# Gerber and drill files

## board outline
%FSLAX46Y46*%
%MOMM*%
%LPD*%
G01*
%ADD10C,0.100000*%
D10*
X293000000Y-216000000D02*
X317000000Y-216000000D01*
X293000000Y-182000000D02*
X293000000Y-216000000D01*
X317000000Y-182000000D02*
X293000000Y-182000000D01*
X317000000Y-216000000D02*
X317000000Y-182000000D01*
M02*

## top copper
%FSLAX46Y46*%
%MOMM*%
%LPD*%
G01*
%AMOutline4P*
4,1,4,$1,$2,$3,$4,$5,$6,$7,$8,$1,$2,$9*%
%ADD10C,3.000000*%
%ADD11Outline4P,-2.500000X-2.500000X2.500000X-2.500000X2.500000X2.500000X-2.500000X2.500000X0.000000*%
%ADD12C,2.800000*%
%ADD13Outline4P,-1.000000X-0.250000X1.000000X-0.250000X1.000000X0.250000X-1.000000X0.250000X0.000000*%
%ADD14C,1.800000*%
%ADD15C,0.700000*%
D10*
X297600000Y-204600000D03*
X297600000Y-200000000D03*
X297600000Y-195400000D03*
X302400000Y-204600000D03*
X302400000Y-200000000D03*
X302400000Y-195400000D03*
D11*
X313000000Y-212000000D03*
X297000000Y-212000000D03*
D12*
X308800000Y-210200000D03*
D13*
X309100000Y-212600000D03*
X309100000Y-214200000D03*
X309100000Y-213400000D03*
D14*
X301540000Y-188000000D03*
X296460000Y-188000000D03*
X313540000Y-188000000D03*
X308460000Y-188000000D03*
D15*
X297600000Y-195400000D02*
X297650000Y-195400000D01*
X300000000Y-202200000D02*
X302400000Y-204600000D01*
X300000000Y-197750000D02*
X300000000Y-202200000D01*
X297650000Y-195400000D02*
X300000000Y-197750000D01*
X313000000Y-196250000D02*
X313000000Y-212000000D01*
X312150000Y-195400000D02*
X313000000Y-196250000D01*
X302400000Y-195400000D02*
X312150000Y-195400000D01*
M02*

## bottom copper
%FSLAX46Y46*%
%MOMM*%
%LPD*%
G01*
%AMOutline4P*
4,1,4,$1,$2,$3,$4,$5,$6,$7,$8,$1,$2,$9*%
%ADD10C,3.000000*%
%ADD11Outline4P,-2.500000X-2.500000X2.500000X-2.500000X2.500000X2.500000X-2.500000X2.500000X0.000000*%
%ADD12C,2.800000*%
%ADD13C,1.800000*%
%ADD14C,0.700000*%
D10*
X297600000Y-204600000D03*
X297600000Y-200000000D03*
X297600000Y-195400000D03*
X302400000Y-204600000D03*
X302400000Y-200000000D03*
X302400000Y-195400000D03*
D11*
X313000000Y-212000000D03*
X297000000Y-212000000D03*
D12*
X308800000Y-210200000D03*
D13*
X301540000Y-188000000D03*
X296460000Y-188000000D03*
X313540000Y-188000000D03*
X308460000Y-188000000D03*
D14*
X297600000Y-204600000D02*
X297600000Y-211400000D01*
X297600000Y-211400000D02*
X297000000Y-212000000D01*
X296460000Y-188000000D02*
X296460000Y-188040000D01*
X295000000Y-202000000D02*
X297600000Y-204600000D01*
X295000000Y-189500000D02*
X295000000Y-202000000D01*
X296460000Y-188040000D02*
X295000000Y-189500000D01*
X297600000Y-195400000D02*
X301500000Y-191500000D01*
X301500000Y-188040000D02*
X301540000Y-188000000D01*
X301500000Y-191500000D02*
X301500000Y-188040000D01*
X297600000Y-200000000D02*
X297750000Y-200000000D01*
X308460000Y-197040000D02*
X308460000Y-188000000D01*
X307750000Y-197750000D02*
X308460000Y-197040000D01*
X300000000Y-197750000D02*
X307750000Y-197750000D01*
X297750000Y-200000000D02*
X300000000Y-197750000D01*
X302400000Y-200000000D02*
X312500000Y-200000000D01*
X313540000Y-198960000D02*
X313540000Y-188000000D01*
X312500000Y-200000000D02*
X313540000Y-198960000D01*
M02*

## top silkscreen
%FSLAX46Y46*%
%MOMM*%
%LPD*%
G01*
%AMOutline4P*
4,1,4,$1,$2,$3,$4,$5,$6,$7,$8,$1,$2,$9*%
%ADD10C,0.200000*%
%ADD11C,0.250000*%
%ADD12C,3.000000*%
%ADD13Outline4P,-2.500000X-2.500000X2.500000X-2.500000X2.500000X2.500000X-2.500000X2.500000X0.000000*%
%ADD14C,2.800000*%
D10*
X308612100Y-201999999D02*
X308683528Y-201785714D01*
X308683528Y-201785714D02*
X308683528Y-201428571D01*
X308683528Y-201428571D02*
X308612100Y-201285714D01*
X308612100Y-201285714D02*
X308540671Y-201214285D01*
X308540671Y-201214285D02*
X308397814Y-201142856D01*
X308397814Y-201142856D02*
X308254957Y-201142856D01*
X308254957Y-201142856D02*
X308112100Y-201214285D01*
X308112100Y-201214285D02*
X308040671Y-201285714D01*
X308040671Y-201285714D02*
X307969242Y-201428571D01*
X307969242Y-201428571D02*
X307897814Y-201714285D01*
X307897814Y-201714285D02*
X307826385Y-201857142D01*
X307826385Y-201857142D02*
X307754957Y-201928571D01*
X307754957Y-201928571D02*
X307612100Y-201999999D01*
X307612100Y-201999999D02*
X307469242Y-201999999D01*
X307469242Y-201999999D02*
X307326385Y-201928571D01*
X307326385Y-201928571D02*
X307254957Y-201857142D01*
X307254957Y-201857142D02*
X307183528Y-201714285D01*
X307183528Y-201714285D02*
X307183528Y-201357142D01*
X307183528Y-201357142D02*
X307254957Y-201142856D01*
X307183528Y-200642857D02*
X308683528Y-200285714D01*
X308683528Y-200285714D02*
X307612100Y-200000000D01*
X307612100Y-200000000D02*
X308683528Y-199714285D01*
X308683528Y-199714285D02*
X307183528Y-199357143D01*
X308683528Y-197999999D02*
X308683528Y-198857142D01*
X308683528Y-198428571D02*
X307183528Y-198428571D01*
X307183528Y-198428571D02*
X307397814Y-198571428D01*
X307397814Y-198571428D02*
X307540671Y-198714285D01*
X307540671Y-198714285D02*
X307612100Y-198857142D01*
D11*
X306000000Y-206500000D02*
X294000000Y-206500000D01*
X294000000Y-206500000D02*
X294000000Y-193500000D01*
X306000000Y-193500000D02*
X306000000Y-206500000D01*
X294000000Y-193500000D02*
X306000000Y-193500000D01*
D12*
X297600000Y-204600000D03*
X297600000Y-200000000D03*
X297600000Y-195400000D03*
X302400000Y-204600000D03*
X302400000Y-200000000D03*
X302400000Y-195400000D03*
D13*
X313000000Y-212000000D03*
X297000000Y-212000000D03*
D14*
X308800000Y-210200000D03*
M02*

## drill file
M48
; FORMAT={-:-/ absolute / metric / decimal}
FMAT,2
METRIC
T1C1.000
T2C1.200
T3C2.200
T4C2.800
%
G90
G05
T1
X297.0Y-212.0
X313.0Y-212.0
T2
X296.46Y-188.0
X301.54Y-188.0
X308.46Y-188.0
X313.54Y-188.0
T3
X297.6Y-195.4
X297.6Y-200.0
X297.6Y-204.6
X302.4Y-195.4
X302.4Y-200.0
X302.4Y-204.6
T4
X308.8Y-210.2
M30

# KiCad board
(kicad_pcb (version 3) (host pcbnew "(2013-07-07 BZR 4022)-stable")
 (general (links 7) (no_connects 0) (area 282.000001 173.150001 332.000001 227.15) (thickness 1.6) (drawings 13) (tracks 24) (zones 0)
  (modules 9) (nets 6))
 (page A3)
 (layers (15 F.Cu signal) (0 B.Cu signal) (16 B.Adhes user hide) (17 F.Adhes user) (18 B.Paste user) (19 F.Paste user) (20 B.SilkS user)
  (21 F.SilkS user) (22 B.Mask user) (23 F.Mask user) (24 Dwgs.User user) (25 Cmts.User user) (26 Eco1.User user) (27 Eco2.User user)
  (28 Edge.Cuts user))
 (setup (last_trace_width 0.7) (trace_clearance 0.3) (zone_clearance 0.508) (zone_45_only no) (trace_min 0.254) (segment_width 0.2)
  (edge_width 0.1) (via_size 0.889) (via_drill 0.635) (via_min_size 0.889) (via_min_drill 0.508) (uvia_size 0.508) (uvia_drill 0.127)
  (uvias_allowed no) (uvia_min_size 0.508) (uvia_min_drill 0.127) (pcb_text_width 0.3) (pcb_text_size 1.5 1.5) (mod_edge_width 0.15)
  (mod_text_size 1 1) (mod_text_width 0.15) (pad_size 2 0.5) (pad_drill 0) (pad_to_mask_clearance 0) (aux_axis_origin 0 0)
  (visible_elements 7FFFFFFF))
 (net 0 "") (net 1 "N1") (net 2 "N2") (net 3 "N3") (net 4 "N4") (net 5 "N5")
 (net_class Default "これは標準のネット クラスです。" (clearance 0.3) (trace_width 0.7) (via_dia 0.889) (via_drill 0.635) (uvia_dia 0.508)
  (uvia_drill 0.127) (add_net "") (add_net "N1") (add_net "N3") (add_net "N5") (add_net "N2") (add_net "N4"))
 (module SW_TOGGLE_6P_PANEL (layer F.Cu) (at 300 200)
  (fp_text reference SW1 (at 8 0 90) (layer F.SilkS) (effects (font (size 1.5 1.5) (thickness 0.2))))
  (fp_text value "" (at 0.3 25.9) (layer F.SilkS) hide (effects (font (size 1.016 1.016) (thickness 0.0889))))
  (fp_line (start 6 6.5) (end -6 6.5) (layer F.SilkS) (width 0.25))
  (fp_line (start -6 6.5) (end -6 -6.5) (layer F.SilkS) (width 0.25))
  (fp_line (start 6 -6.5) (end 6 6.5) (layer F.SilkS) (width 0.25))
  (fp_line (start -6 -6.5) (end 6 -6.5) (layer F.SilkS) (width 0.25))
  (pad 1 thru_hole circle (at -2.4 4.6) (size 3 3) (drill 2.2) (layers *.Cu *.Mask F.SilkS) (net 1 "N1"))
  (pad 2 thru_hole circle (at -2.4 0) (size 3 3) (drill 2.2) (layers *.Cu *.Mask F.SilkS) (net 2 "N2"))
  (pad 3 thru_hole circle (at -2.4 -4.6) (size 3 3) (drill 2.2) (layers *.Cu *.Mask F.SilkS) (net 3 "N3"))
  (pad 4 thru_hole circle (at 2.4 4.6) (size 3 3) (drill 2.2) (layers *.Cu *.Mask F.SilkS) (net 3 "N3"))
  (pad 5 thru_hole circle (at 2.4 0) (size 3 3) (drill 2.2) (layers *.Cu *.Mask F.SilkS) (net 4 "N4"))
  (pad 6 thru_hole circle (at 2.4 -4.6) (size 3 3) (drill 2.2) (layers *.Cu *.Mask F.SilkS) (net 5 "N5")))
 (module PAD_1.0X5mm (layer F.Cu) (at 313 212)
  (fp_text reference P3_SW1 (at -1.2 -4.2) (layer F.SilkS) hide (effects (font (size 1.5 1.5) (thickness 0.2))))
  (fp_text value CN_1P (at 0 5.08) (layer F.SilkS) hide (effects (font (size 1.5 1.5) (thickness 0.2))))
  (pad 1 thru_hole trapezoid (at 0 0) (size 5 5) (drill 1) (layers *.Cu *.Mask F.SilkS) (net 5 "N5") (clearance 0.3)))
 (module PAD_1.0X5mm (layer F.Cu) (at 297 212)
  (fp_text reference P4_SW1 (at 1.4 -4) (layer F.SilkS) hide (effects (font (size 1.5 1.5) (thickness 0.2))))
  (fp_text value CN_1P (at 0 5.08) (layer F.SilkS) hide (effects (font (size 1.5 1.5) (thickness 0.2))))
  (pad 1 thru_hole trapezoid (at 0 0) (size 5 5) (drill 1) (layers *.Cu *.Mask F.SilkS) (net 1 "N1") (clearance 0.3)))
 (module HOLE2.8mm (layer F.Cu) (at 308.8 210.2)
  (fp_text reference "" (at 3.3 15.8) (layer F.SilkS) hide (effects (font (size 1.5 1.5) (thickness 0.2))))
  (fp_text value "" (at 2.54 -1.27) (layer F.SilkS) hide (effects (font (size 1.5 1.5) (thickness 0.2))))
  (pad "" thru_hole circle (at 0 0) (size 2.8 2.8) (drill 2.8) (layers *.Cu *.Mask F.SilkS) (clearance 0.3)))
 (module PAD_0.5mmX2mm (layer F.Cu) (at 309.1 212.6)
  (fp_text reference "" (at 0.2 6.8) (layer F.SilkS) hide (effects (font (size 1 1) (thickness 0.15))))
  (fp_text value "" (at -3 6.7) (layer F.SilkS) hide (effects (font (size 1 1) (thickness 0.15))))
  (pad 1 smd trapezoid (at 0 0) (size 2 0.5) (layers F.Cu F.Paste F.Mask)))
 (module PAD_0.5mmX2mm (layer F.Cu) (at 309.1 214.2)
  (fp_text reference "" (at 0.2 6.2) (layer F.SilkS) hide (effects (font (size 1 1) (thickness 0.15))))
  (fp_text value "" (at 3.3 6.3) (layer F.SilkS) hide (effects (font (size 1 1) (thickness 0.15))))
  (pad 1 smd trapezoid (at 0 0) (size 2 0.5) (layers F.Cu F.Paste F.Mask)))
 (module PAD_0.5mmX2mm (layer F.Cu) (at 309.1 213.4)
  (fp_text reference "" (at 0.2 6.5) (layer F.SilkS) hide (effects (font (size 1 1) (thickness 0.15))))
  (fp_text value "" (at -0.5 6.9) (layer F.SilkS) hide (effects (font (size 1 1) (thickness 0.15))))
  (pad 1 smd trapezoid (at 0 0) (size 2 0.5) (layers F.Cu F.Paste F.Mask)))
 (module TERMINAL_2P (layer B.Cu) (at 299 188 180)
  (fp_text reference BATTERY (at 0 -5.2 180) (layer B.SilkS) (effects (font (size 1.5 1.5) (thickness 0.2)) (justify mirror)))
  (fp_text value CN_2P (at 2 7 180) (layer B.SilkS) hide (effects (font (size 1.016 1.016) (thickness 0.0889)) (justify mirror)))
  (pad 1 thru_hole circle (at -2.54 0 180) (size 1.8 1.8) (drill 1.2) (layers *.Cu *.Mask B.SilkS) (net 3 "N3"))
  (pad 2 thru_hole circle (at 2.54 0 180) (size 1.8 1.8) (drill 1.2) (layers *.Cu *.Mask B.SilkS) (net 1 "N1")))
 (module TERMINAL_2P (layer B.Cu) (at 311 188 180)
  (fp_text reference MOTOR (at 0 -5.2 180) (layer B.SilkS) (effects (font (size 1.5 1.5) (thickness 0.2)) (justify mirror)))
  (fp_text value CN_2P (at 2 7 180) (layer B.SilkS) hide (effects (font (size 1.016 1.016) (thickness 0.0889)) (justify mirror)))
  (pad 1 thru_hole circle (at -2.54 0 180) (size 1.8 1.8) (drill 1.2) (layers *.Cu *.Mask B.SilkS) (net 4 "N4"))
  (pad 2 thru_hole circle (at 2.54 0 180) (size 1.8 1.8) (drill 1.2) (layers *.Cu *.Mask B.SilkS) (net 2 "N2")))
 (gr_line (start 293 216) (end 317 216) (angle 90) (layer Edge.Cuts) (width 0.1))
 (gr_line (start 293 182) (end 293 216) (angle 90) (layer Edge.Cuts) (width 0.1))
 (gr_line (start 317 182) (end 293 182) (angle 90) (layer Edge.Cuts) (width 0.1))
 (gr_line (start 317 216) (end 317 182) (angle 90) (layer Edge.Cuts) (width 0.1))
 (segment (start 297.6 204.6) (end 297.6 211.4) (width 0.7) (layer B.Cu) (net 1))
 (segment (start 297.6 211.4) (end 297 212) (width 0.7) (layer B.Cu) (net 1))
 (segment (start 296.46 188) (end 296.46 188.04) (width 0.7) (layer B.Cu) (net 1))
 (segment (start 295 202) (end 297.6 204.6) (width 0.7) (layer B.Cu) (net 1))
 (segment (start 295 189.5) (end 295 202) (width 0.7) (layer B.Cu) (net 1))
 (segment (start 296.46 188.04) (end 295 189.5) (width 0.7) (layer B.Cu) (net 1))
 (segment (start 297.6 195.4) (end 297.65 195.4) (width 0.7) (layer F.Cu) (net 3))
 (segment (start 300 202.2) (end 302.4 204.6) (width 0.7) (layer F.Cu) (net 3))
 (segment (start 300 197.75) (end 300 202.2) (width 0.7) (layer F.Cu) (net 3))
 (segment (start 297.65 195.4) (end 300 197.75) (width 0.7) (layer F.Cu) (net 3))
 (segment (start 297.6 195.4) (end 301.5 191.5) (width 0.7) (layer B.Cu) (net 3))
 (segment (start 301.5 188.04) (end 301.54 188) (width 0.7) (layer B.Cu) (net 3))
 (segment (start 301.5 191.5) (end 301.5 188.04) (width 0.7) (layer B.Cu) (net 3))
 (segment (start 313 196.25) (end 313 212) (width 0.7) (layer F.Cu) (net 5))
 (segment (start 312.15 195.4) (end 313 196.25) (width 0.7) (layer F.Cu) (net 5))
 (segment (start 302.4 195.4) (end 312.15 195.4) (width 0.7) (layer F.Cu) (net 5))
 (segment (start 297.6 200) (end 297.75 200) (width 0.7) (layer B.Cu) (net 2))
 (segment (start 308.46 197.04) (end 308.46 188) (width 0.7) (layer B.Cu) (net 2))
 (segment (start 307.75 197.75) (end 308.46 197.04) (width 0.7) (layer B.Cu) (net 2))
 (segment (start 300 197.75) (end 307.75 197.75) (width 0.7) (layer B.Cu) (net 2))
 (segment (start 297.75 200) (end 300 197.75) (width 0.7) (layer B.Cu) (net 2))
 (segment (start 302.4 200) (end 312.5 200) (width 0.7) (layer B.Cu) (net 4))
 (segment (start 313.54 198.96) (end 313.54 188) (width 0.7) (layer B.Cu) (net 4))
 (segment (start 312.5 200) (end 313.54 198.96) (width 0.7) (layer B.Cu) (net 4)))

